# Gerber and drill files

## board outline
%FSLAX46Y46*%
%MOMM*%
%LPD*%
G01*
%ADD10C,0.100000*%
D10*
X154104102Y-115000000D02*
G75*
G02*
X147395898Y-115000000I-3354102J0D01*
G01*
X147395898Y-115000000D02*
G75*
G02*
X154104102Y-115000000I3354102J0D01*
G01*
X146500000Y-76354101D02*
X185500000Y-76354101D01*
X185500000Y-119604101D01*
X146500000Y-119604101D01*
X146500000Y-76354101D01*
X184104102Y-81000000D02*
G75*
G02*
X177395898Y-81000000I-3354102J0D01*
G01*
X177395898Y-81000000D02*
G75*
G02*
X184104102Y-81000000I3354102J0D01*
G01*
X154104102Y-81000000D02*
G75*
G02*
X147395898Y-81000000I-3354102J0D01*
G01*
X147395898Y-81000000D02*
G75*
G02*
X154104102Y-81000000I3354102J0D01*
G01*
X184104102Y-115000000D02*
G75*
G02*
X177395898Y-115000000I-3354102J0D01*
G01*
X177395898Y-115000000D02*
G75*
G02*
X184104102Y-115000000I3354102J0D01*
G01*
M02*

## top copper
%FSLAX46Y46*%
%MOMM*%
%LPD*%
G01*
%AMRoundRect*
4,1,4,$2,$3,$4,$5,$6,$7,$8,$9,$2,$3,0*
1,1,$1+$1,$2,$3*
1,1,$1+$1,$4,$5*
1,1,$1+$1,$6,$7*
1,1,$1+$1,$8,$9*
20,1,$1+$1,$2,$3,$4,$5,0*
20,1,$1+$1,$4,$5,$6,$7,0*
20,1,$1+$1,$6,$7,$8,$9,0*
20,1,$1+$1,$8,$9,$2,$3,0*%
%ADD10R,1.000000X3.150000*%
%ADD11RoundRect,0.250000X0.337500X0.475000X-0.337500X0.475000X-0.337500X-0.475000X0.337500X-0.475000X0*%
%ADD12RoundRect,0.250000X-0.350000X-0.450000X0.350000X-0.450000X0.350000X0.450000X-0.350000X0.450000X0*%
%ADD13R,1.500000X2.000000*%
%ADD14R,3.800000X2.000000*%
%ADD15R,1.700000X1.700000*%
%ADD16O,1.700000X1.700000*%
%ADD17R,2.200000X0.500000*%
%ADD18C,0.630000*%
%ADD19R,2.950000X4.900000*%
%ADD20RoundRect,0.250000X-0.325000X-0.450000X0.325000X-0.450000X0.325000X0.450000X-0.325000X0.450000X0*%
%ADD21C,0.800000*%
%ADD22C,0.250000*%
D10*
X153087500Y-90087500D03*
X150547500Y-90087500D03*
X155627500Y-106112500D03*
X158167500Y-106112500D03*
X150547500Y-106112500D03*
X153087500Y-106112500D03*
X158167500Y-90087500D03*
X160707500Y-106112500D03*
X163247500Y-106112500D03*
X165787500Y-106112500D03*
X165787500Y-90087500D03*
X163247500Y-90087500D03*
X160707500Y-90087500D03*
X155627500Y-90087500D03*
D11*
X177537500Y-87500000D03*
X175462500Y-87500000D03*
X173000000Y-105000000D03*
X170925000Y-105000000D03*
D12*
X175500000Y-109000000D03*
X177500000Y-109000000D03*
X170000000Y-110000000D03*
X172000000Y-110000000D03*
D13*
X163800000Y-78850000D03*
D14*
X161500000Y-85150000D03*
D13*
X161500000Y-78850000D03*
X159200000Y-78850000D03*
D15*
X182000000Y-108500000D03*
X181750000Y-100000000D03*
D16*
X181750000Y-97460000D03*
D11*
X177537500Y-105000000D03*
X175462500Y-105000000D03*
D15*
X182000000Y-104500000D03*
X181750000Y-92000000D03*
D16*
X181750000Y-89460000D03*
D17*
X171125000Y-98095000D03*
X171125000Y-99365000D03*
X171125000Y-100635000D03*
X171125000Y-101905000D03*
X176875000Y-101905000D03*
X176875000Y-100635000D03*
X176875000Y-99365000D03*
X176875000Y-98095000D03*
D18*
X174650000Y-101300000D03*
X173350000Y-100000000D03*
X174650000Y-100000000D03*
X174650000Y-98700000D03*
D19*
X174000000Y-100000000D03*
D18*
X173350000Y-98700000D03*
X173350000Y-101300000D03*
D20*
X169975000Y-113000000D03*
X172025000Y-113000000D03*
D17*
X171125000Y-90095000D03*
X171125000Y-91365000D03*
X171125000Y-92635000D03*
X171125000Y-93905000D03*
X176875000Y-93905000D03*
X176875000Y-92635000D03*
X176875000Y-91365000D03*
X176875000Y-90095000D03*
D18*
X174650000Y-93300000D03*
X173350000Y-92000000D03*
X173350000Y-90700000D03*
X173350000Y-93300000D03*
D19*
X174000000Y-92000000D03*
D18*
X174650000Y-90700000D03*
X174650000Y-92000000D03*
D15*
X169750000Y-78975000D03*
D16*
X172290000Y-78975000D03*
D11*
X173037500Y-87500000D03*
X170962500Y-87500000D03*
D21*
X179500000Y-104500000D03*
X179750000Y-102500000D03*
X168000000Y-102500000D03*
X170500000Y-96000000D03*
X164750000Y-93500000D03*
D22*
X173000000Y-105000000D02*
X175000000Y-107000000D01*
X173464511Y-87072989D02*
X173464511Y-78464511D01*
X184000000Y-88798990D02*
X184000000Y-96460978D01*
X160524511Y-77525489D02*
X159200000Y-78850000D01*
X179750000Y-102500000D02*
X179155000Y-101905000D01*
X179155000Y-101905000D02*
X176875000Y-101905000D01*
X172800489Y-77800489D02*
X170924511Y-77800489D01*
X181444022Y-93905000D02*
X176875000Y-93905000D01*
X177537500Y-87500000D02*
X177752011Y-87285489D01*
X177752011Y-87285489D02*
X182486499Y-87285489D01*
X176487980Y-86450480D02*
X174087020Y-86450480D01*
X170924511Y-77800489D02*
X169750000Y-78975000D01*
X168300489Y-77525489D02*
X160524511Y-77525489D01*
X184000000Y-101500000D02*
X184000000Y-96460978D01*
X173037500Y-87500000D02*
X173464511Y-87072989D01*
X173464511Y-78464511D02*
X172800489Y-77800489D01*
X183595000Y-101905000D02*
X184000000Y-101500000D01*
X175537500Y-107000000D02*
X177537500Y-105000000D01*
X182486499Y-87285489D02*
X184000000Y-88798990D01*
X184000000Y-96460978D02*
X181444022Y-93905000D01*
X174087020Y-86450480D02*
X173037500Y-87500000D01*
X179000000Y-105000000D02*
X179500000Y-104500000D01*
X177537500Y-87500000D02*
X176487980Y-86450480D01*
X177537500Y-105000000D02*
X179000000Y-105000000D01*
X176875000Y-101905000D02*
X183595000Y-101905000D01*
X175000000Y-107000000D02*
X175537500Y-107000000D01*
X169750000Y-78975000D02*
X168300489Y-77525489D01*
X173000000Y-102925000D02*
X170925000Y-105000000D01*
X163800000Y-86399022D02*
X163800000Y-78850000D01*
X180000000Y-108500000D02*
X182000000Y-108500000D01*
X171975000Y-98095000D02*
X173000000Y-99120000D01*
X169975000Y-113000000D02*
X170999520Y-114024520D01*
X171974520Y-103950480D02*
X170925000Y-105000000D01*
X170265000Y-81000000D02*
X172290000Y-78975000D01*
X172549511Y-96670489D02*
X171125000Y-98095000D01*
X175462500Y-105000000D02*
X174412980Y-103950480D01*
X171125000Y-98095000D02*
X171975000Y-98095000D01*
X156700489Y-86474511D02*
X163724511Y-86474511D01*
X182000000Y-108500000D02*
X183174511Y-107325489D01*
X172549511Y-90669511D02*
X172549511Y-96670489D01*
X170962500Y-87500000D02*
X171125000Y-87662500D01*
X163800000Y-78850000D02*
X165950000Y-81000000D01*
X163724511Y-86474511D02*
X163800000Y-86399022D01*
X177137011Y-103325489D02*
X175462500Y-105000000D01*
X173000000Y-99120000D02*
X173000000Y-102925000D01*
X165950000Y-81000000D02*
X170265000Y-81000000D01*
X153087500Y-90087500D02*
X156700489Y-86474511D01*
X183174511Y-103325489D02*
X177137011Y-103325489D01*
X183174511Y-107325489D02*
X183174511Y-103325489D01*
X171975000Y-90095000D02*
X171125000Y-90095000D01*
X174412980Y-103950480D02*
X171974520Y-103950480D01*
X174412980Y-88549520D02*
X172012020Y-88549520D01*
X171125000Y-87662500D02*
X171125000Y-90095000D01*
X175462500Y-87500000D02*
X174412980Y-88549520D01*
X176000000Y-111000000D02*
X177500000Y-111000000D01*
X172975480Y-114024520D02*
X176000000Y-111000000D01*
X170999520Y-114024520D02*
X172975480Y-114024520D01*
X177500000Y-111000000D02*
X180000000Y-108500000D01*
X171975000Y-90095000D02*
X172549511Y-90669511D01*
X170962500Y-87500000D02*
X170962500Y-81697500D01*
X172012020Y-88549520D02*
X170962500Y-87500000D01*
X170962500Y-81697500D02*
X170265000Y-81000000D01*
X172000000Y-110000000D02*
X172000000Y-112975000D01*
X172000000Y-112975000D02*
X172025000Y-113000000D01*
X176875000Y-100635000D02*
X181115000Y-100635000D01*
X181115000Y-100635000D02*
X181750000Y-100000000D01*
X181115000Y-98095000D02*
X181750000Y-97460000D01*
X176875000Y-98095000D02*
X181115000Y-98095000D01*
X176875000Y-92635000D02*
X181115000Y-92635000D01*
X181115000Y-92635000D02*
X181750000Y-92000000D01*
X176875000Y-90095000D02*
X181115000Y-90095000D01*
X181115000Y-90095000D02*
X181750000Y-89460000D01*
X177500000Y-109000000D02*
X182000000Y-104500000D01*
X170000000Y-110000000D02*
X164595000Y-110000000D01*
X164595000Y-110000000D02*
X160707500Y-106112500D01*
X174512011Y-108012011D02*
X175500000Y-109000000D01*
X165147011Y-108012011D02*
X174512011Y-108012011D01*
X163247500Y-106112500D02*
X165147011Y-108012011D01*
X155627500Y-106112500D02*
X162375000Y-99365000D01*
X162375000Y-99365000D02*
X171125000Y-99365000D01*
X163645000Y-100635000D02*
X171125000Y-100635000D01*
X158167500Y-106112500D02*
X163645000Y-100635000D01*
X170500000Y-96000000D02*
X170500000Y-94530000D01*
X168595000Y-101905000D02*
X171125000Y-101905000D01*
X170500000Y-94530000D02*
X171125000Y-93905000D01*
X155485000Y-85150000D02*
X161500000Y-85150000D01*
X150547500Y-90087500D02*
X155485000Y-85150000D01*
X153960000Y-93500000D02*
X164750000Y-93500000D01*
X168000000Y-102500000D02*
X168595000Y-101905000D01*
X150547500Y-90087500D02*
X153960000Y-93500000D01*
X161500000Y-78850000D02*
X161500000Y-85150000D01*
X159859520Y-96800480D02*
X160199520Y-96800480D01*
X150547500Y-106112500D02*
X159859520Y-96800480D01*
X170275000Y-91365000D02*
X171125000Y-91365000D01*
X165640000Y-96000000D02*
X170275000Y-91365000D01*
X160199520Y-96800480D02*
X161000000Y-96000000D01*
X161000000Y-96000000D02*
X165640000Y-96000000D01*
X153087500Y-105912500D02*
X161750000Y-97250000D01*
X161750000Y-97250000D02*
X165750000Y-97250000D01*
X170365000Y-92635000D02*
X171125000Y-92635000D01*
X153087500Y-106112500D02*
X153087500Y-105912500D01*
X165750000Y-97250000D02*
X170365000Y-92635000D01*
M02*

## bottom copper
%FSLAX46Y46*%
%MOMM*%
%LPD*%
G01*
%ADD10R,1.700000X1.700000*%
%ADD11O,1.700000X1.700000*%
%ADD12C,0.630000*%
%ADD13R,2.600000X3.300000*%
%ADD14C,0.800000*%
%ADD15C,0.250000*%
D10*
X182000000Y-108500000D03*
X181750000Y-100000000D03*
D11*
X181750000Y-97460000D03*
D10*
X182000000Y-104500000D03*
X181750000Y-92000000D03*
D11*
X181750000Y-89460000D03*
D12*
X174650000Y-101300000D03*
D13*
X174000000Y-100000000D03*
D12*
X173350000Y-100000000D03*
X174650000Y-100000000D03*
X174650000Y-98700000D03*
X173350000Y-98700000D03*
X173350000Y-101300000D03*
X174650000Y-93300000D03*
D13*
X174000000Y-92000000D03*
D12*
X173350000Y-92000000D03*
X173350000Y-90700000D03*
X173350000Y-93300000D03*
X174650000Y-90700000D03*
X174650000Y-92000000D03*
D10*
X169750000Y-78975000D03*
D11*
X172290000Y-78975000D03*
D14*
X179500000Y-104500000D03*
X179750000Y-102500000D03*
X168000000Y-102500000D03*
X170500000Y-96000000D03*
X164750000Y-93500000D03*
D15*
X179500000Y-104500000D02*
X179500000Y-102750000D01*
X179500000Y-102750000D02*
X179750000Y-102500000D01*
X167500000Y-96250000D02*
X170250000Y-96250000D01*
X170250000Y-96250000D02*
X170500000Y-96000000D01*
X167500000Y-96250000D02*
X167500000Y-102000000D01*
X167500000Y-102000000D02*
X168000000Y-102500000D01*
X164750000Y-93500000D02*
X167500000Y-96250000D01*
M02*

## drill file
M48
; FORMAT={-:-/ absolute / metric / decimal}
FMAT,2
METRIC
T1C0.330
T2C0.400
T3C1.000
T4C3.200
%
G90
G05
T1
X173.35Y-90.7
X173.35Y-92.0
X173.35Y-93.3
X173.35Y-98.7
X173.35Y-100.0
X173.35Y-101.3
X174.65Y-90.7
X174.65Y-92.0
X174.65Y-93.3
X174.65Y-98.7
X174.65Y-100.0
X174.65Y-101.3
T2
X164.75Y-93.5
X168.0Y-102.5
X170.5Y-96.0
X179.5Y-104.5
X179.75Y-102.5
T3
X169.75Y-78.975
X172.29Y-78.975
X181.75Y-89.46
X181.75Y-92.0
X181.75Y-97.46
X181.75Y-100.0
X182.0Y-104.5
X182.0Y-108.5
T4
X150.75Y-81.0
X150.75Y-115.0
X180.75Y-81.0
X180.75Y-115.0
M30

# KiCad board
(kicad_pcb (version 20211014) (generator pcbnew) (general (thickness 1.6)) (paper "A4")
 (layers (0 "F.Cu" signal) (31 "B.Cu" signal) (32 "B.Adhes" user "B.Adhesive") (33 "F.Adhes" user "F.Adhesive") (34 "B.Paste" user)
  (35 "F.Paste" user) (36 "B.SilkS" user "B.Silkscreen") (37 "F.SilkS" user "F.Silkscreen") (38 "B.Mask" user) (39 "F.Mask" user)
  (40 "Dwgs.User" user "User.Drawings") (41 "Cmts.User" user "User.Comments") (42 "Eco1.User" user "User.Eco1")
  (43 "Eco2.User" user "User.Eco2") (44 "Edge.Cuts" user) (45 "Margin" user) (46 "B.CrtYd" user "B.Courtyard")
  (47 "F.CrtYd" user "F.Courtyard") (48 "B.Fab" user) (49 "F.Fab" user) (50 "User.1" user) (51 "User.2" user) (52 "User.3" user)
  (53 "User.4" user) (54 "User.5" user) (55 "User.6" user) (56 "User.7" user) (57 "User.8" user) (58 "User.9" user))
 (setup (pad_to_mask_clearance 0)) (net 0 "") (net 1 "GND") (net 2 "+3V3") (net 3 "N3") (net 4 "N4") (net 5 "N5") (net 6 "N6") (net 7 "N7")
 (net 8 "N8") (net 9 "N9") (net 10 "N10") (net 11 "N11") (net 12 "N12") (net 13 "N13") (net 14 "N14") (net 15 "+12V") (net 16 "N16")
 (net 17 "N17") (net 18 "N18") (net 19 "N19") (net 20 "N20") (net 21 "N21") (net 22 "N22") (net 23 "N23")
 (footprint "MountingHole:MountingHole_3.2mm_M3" (layer "F.Cu") (at 180.75 115)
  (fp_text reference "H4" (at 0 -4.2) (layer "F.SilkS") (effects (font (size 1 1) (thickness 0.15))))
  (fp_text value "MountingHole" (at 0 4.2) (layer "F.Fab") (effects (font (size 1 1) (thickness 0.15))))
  (pad "" np_thru_hole circle (at 0 0) (size 3.2 3.2) (drill 3.2) (layers *.Cu *.Mask)))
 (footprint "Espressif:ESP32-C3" (layer "F.Cu") (at 159.9675 97.5125 90)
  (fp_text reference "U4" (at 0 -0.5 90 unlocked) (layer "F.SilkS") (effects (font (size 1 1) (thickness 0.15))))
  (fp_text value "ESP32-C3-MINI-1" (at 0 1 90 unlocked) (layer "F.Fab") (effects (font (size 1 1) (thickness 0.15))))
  (pad "1" smd rect (at 7.425 -6.88 90) (size 3.15 1) (layers "F.Cu" "F.Paste" "F.Mask") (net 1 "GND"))
  (pad "3" smd rect (at 7.425 -9.42 90) (size 3.15 1) (layers "F.Cu" "F.Paste" "F.Mask") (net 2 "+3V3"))
  (pad "5" smd rect (at -8.6 -4.34 90) (size 3.15 1) (layers "F.Cu" "F.Paste" "F.Mask") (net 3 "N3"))
  (pad "6" smd rect (at -8.6 -1.8 90) (size 3.15 1) (layers "F.Cu" "F.Paste" "F.Mask") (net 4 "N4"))
  (pad "12" smd rect (at -8.6 -9.42 90) (size 3.15 1) (layers "F.Cu" "F.Paste" "F.Mask") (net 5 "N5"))
  (pad "13" smd rect (at -8.6 -6.88 90) (size 3.15 1) (layers "F.Cu" "F.Paste" "F.Mask") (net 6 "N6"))
  (pad "16" smd rect (at 7.425 -1.8 90) (size 3.15 1) (layers "F.Cu" "F.Paste" "F.Mask") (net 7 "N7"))
  (pad "18" smd rect (at -8.6 0.74 90) (size 3.15 1) (layers "F.Cu" "F.Paste" "F.Mask") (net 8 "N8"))
  (pad "19" smd rect (at -8.6 3.28 90) (size 3.15 1) (layers "F.Cu" "F.Paste" "F.Mask") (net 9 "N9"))
  (pad "20" smd rect (at -8.6 5.82 90) (size 3.15 1) (layers "F.Cu" "F.Paste" "F.Mask") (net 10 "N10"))
  (pad "21" smd rect (at 7.425 5.82 90) (size 3.15 1) (layers "F.Cu" "F.Paste" "F.Mask") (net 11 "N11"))
  (pad "22" smd rect (at 7.425 3.28 90) (size 3.15 1) (layers "F.Cu" "F.Paste" "F.Mask") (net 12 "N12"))
  (pad "23" smd rect (at 7.425 0.74 90) (size 3.15 1) (layers "F.Cu" "F.Paste" "F.Mask") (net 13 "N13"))
  (pad "35" smd rect (at 7.425 -4.34 90) (size 3.15 1) (layers "F.Cu" "F.Paste" "F.Mask") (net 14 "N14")))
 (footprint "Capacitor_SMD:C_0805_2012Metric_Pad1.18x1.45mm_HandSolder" (layer "F.Cu") (at 176.5 87.5 180)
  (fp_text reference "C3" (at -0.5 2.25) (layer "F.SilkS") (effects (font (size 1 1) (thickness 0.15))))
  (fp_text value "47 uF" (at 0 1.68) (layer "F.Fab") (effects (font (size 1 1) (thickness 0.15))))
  (pad "1" smd roundrect (at -1.0375 0 180) (size 1.175 1.45) (layers "F.Cu" "F.Paste" "F.Mask") (roundrect_rratio 0.2127659574)
   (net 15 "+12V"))
  (pad "2" smd roundrect (at 1.0375 0 180) (size 1.175 1.45) (layers "F.Cu" "F.Paste" "F.Mask") (roundrect_rratio 0.2127659574)
   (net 1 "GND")))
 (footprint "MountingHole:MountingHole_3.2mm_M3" (layer "F.Cu") (at 180.75 81)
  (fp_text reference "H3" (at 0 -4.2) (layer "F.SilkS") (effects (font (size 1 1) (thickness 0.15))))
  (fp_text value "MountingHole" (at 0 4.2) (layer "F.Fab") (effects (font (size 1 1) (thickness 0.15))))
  (pad "" np_thru_hole circle (at 0 0) (size 3.2 3.2) (drill 3.2) (layers *.Cu *.Mask)))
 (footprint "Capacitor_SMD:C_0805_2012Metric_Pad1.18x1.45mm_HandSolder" (layer "F.Cu") (at 171.9625 105 180)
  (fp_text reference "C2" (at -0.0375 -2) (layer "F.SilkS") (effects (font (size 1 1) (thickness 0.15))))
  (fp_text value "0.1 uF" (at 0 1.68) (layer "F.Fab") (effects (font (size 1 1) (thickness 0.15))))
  (pad "1" smd roundrect (at -1.0375 0 180) (size 1.175 1.45) (layers "F.Cu" "F.Paste" "F.Mask") (roundrect_rratio 0.2127659574)
   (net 15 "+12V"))
  (pad "2" smd roundrect (at 1.0375 0 180) (size 1.175 1.45) (layers "F.Cu" "F.Paste" "F.Mask") (roundrect_rratio 0.2127659574)
   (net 1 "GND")))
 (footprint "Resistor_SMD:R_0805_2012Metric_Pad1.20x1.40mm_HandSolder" (layer "F.Cu") (at 176.5 109)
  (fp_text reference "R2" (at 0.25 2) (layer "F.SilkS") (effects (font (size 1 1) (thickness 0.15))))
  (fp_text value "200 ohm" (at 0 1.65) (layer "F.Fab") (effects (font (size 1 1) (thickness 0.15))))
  (pad "1" smd roundrect (at -1 0) (size 1.2 1.4) (layers "F.Cu" "F.Paste" "F.Mask") (roundrect_rratio 0.2083333333) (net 9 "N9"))
  (pad "2" smd roundrect (at 1 0) (size 1.2 1.4) (layers "F.Cu" "F.Paste" "F.Mask") (roundrect_rratio 0.2083333333) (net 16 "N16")))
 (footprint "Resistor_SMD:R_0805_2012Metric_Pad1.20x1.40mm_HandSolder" (layer "F.Cu") (at 171 110)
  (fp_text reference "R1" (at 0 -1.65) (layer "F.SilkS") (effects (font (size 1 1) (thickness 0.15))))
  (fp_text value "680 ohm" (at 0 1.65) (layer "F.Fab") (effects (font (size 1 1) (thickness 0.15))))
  (pad "1" smd roundrect (at -1 0) (size 1.2 1.4) (layers "F.Cu" "F.Paste" "F.Mask") (roundrect_rratio 0.2083333333) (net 8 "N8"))
  (pad "2" smd roundrect (at 1 0) (size 1.2 1.4) (layers "F.Cu" "F.Paste" "F.Mask") (roundrect_rratio 0.2083333333) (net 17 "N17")))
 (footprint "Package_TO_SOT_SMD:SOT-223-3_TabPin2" (layer "F.Cu") (at 161.5 82 -90)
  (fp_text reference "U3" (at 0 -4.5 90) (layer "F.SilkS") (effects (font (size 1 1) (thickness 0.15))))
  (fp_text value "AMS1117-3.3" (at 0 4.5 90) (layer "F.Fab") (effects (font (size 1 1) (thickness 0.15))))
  (pad "1" smd rect (at -3.15 -2.3 270) (size 2 1.5) (layers "F.Cu" "F.Paste" "F.Mask") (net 1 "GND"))
  (pad "2" smd rect (at 3.15 0 270) (size 2 3.8) (layers "F.Cu" "F.Paste" "F.Mask") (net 2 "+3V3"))
  (pad "2" smd rect (at -3.15 0 270) (size 2 1.5) (layers "F.Cu" "F.Paste" "F.Mask") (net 2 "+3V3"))
  (pad "3" smd rect (at -3.15 2.3 270) (size 2 1.5) (layers "F.Cu" "F.Paste" "F.Mask") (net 15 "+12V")))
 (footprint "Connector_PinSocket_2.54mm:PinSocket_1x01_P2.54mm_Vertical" (layer "F.Cu") (at 182 108.5 180)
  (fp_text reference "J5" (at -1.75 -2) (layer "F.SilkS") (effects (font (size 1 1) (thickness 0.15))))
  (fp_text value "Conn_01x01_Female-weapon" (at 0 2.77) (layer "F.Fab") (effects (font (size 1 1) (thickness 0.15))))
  (pad "1" thru_hole rect (at 0 0 180) (size 1.7 1.7) (drill 1) (layers *.Cu *.Mask) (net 1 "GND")))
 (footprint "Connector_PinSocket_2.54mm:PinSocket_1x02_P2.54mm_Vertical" (layer "F.Cu") (at 181.75 100 180)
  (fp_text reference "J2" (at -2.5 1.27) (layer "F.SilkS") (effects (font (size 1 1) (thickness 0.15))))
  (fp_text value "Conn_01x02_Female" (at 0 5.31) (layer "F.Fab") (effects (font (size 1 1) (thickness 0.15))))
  (pad "1" thru_hole rect (at 0 0 180) (size 1.7 1.7) (drill 1) (layers *.Cu *.Mask) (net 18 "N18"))
  (pad "2" thru_hole oval (at 0 2.54 180) (size 1.7 1.7) (drill 1) (layers *.Cu *.Mask) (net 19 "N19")))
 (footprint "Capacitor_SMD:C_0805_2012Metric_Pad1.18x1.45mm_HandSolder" (layer "F.Cu") (at 176.5 105 180)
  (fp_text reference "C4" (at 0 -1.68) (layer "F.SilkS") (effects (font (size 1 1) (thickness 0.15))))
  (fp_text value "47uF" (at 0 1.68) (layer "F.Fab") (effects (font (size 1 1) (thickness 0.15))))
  (pad "1" smd roundrect (at -1.0375 0 180) (size 1.175 1.45) (layers "F.Cu" "F.Paste" "F.Mask") (roundrect_rratio 0.2127659574)
   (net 15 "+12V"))
  (pad "2" smd roundrect (at 1.0375 0 180) (size 1.175 1.45) (layers "F.Cu" "F.Paste" "F.Mask") (roundrect_rratio 0.2127659574)
   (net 1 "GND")))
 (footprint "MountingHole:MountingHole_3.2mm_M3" (layer "F.Cu") (at 150.75 115)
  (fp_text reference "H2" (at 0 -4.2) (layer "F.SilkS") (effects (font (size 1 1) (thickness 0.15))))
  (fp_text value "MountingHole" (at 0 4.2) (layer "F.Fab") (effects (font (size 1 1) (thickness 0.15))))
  (pad "" np_thru_hole circle (at 0 0) (size 3.2 3.2) (drill 3.2) (layers *.Cu *.Mask)))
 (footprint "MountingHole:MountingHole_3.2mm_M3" (layer "F.Cu") (at 150.75 81)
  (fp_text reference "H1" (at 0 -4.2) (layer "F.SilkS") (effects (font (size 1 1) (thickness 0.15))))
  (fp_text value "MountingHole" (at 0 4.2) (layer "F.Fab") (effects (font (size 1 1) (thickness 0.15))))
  (pad "" np_thru_hole circle (at 0 0) (size 3.2 3.2) (drill 3.2) (layers *.Cu *.Mask)))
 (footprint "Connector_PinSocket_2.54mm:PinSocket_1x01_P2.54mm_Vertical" (layer "F.Cu") (at 182 104.5)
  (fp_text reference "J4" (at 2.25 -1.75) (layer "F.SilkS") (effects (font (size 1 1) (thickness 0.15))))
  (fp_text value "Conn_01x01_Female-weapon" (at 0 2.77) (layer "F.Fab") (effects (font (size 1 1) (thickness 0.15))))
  (pad "1" thru_hole rect (at 0 0) (size 1.7 1.7) (drill 1) (layers *.Cu *.Mask) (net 16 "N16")))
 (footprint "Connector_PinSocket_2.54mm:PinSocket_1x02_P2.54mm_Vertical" (layer "F.Cu") (at 181.75 92 180)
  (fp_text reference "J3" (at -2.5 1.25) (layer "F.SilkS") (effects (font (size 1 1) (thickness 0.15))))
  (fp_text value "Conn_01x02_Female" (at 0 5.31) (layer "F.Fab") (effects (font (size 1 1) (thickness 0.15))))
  (pad "1" thru_hole rect (at 0 0 180) (size 1.7 1.7) (drill 1) (layers *.Cu *.Mask) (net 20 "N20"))
  (pad "2" thru_hole oval (at 0 2.54 180) (size 1.7 1.7) (drill 1) (layers *.Cu *.Mask) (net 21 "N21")))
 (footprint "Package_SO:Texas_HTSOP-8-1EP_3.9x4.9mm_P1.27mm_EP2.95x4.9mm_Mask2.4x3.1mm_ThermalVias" (layer "F.Cu") (at 174 100)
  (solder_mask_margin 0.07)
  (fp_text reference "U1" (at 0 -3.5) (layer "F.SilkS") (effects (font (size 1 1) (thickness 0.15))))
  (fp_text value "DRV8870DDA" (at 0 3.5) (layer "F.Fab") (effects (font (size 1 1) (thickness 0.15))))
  (pad "" smd rect (at 0 0) (size 2.4 3.1) (layers "F.Paste")) (pad "" smd rect (at 0 0) (size 2.4 3.1) (layers "F.Mask"))
  (pad "1" smd rect (at -2.875 -1.905) (size 2.2 0.5) (layers "F.Cu" "F.Paste" "F.Mask") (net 1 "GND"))
  (pad "2" smd rect (at -2.875 -0.635) (size 2.2 0.5) (layers "F.Cu" "F.Paste" "F.Mask") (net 3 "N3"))
  (pad "3" smd rect (at -2.875 0.635) (size 2.2 0.5) (layers "F.Cu" "F.Paste" "F.Mask") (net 4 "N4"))
  (pad "4" smd rect (at -2.875 1.905) (size 2.2 0.5) (layers "F.Cu" "F.Paste" "F.Mask") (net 2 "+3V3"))
  (pad "5" smd rect (at 2.875 1.905) (size 2.2 0.5) (layers "F.Cu" "F.Paste" "F.Mask") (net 15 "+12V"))
  (pad "6" smd rect (at 2.875 0.635) (size 2.2 0.5) (layers "F.Cu" "F.Paste" "F.Mask") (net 18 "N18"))
  (pad "7" smd rect (at 2.875 -0.635) (size 2.2 0.5) (layers "F.Cu" "F.Paste" "F.Mask") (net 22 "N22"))
  (pad "8" smd rect (at 2.875 -1.905) (size 2.2 0.5) (layers "F.Cu" "F.Paste" "F.Mask") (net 19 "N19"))
  (pad "9" thru_hole circle (at 0.65 1.3) (size 0.63 0.63) (drill 0.33) (layers *.Cu *.Mask) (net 1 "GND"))
  (pad "9" smd rect (at 0 0) (size 2.6 3.3) (layers "B.Cu") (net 1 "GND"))
  (pad "9" thru_hole circle (at -0.65 0) (size 0.63 0.63) (drill 0.33) (layers *.Cu *.Mask) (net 1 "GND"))
  (pad "9" thru_hole circle (at 0.65 0) (size 0.63 0.63) (drill 0.33) (layers *.Cu *.Mask) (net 1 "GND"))
  (pad "9" thru_hole circle (at 0.65 -1.3) (size 0.63 0.63) (drill 0.33) (layers *.Cu *.Mask) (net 1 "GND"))
  (pad "9" smd rect (at 0 0) (size 2.95 4.9) (layers "F.Cu") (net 1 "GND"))
  (pad "9" thru_hole circle (at -0.65 -1.3) (size 0.63 0.63) (drill 0.33) (layers *.Cu *.Mask) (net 1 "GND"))
  (pad "9" thru_hole circle (at -0.65 1.3) (size 0.63 0.63) (drill 0.33) (layers *.Cu *.Mask) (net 1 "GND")))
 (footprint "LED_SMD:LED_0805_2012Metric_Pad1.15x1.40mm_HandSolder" (layer "F.Cu") (at 171 113)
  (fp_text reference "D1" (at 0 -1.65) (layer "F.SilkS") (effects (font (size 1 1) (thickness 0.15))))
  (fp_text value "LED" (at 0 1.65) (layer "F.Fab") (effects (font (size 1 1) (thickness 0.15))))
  (pad "1" smd roundrect (at -1.025 0) (size 1.15 1.4) (layers "F.Cu" "F.Paste" "F.Mask") (roundrect_rratio 0.2173913043) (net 1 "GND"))
  (pad "2" smd roundrect (at 1.025 0) (size 1.15 1.4) (layers "F.Cu" "F.Paste" "F.Mask") (roundrect_rratio 0.2173913043) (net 17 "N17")))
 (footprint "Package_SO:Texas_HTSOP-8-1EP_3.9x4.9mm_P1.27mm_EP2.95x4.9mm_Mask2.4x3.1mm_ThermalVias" (layer "F.Cu") (at 174 92)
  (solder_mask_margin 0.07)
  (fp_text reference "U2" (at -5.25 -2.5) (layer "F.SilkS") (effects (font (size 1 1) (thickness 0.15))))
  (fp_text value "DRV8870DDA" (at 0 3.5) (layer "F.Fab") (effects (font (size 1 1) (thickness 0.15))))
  (pad "" smd rect (at 0 0) (size 2.4 3.1) (layers "F.Mask")) (pad "" smd rect (at 0 0) (size 2.4 3.1) (layers "F.Paste"))
  (pad "1" smd rect (at -2.875 -1.905) (size 2.2 0.5) (layers "F.Cu" "F.Paste" "F.Mask") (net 1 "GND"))
  (pad "2" smd rect (at -2.875 -0.635) (size 2.2 0.5) (layers "F.Cu" "F.Paste" "F.Mask") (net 5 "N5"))
  (pad "3" smd rect (at -2.875 0.635) (size 2.2 0.5) (layers "F.Cu" "F.Paste" "F.Mask") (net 6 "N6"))
  (pad "4" smd rect (at -2.875 1.905) (size 2.2 0.5) (layers "F.Cu" "F.Paste" "F.Mask") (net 2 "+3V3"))
  (pad "5" smd rect (at 2.875 1.905) (size 2.2 0.5) (layers "F.Cu" "F.Paste" "F.Mask") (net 15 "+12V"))
  (pad "6" smd rect (at 2.875 0.635) (size 2.2 0.5) (layers "F.Cu" "F.Paste" "F.Mask") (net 20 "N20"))
  (pad "7" smd rect (at 2.875 -0.635) (size 2.2 0.5) (layers "F.Cu" "F.Paste" "F.Mask") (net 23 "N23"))
  (pad "8" smd rect (at 2.875 -1.905) (size 2.2 0.5) (layers "F.Cu" "F.Paste" "F.Mask") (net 21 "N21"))
  (pad "9" thru_hole circle (at 0.65 1.3) (size 0.63 0.63) (drill 0.33) (layers *.Cu *.Mask) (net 1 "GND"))
  (pad "9" smd rect (at 0 0) (size 2.6 3.3) (layers "B.Cu") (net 1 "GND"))
  (pad "9" thru_hole circle (at -0.65 0) (size 0.63 0.63) (drill 0.33) (layers *.Cu *.Mask) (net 1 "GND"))
  (pad "9" thru_hole circle (at -0.65 -1.3) (size 0.63 0.63) (drill 0.33) (layers *.Cu *.Mask) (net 1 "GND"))
  (pad "9" thru_hole circle (at -0.65 1.3) (size 0.63 0.63) (drill 0.33) (layers *.Cu *.Mask) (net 1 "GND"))
  (pad "9" smd rect (at 0 0) (size 2.95 4.9) (layers "F.Cu") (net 1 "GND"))
  (pad "9" thru_hole circle (at 0.65 -1.3) (size 0.63 0.63) (drill 0.33) (layers *.Cu *.Mask) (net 1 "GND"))
  (pad "9" thru_hole circle (at 0.65 0) (size 0.63 0.63) (drill 0.33) (layers *.Cu *.Mask) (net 1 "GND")))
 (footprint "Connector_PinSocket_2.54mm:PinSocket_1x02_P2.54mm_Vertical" (layer "F.Cu") (at 169.75 78.975 90)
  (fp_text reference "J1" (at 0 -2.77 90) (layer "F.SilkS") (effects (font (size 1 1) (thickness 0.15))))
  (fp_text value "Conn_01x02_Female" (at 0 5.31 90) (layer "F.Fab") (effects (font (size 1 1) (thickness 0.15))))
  (pad "1" thru_hole rect (at 0 0 90) (size 1.7 1.7) (drill 1) (layers *.Cu *.Mask) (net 15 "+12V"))
  (pad "2" thru_hole oval (at 0 2.54 90) (size 1.7 1.7) (drill 1) (layers *.Cu *.Mask) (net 1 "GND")))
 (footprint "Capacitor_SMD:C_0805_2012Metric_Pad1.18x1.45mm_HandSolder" (layer "F.Cu") (at 172 87.5 180)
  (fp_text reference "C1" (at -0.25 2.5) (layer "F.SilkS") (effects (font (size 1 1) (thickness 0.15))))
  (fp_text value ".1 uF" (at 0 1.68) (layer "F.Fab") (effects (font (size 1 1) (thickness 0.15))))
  (pad "1" smd roundrect (at -1.0375 0 180) (size 1.175 1.45) (layers "F.Cu" "F.Paste" "F.Mask") (roundrect_rratio 0.2127659574)
   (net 15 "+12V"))
  (pad "2" smd roundrect (at 1.0375 0 180) (size 1.175 1.45) (layers "F.Cu" "F.Paste" "F.Mask") (roundrect_rratio 0.2127659574)
   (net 1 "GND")))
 (gr_circle (center 150.75 115) (end 153.75 116.5) (layer "Edge.Cuts") (width 0.1) (fill none))
 (gr_rect (start 146.5 76.354101) (end 185.5 119.604101) (layer "Edge.Cuts") (width 0.1) (fill none))
 (gr_circle (center 180.75 81) (end 183.75 82.5) (layer "Edge.Cuts") (width 0.1) (fill none))
 (gr_circle (center 150.75 81) (end 153.75 82.5) (layer "Edge.Cuts") (width 0.1) (fill none))
 (gr_circle (center 180.75 115) (end 183.75 116.5) (layer "Edge.Cuts") (width 0.1) (fill none))
 (segment (start 173 105) (end 175 107) (width 0.25) (layer "F.Cu") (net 15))
 (segment (start 173.464511 87.072989) (end 173.464511 78.464511) (width 0.25) (layer "F.Cu") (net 15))
 (segment (start 184 88.79899) (end 184 96.460978) (width 0.25) (layer "F.Cu") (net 15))
 (segment (start 160.524511 77.525489) (end 159.2 78.85) (width 0.25) (layer "F.Cu") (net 15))
 (segment (start 179.75 102.5) (end 179.155 101.905) (width 0.25) (layer "F.Cu") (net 15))
 (segment (start 179.155 101.905) (end 176.875 101.905) (width 0.25) (layer "F.Cu") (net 15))
 (segment (start 172.800489 77.800489) (end 170.924511 77.800489) (width 0.25) (layer "F.Cu") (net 15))
 (segment (start 181.444022 93.905) (end 176.875 93.905) (width 0.25) (layer "F.Cu") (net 15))
 (segment (start 177.5375 87.5) (end 177.752011 87.285489) (width 0.25) (layer "F.Cu") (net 15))
 (segment (start 177.752011 87.285489) (end 182.486499 87.285489) (width 0.25) (layer "F.Cu") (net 15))
 (segment (start 176.48798 86.45048) (end 174.08702 86.45048) (width 0.25) (layer "F.Cu") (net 15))
 (segment (start 170.924511 77.800489) (end 169.75 78.975) (width 0.25) (layer "F.Cu") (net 15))
 (segment (start 168.300489 77.525489) (end 160.524511 77.525489) (width 0.25) (layer "F.Cu") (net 15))
 (segment (start 184 101.5) (end 184 96.460978) (width 0.25) (layer "F.Cu") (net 15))
 (segment (start 173.0375 87.5) (end 173.464511 87.072989) (width 0.25) (layer "F.Cu") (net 15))
 (segment (start 173.464511 78.464511) (end 172.800489 77.800489) (width 0.25) (layer "F.Cu") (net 15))
 (segment (start 183.595 101.905) (end 184 101.5) (width 0.25) (layer "F.Cu") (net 15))
 (segment (start 175.5375 107) (end 177.5375 105) (width 0.25) (layer "F.Cu") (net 15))
 (segment (start 182.486499 87.285489) (end 184 88.79899) (width 0.25) (layer "F.Cu") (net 15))
 (segment (start 184 96.460978) (end 181.444022 93.905) (width 0.25) (layer "F.Cu") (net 15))
 (segment (start 174.08702 86.45048) (end 173.0375 87.5) (width 0.25) (layer "F.Cu") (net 15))
 (segment (start 179 105) (end 179.5 104.5) (width 0.25) (layer "F.Cu") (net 15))
 (segment (start 177.5375 87.5) (end 176.48798 86.45048) (width 0.25) (layer "F.Cu") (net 15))
 (segment (start 177.5375 105) (end 179 105) (width 0.25) (layer "F.Cu") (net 15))
 (segment (start 176.875 101.905) (end 183.595 101.905) (width 0.25) (layer "F.Cu") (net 15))
 (segment (start 175 107) (end 175.5375 107) (width 0.25) (layer "F.Cu") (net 15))
 (segment (start 169.75 78.975) (end 168.300489 77.525489) (width 0.25) (layer "F.Cu") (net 15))
 (via (at 179.5 104.5) (size 0.8) (drill 0.4) (layers "F.Cu" "B.Cu") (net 15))
 (via (at 179.75 102.5) (size 0.8) (drill 0.4) (layers "F.Cu" "B.Cu") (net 15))
 (segment (start 179.5 104.5) (end 179.5 102.75) (width 0.25) (layer "B.Cu") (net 15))
 (segment (start 179.5 102.75) (end 179.75 102.5) (width 0.25) (layer "B.Cu") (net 15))
 (segment (start 173 102.925) (end 170.925 105) (width 0.25) (layer "F.Cu") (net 1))
 (segment (start 163.8 86.399022) (end 163.8 78.85) (width 0.25) (layer "F.Cu") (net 1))
 (segment (start 180 108.5) (end 182 108.5) (width 0.25) (layer "F.Cu") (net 1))
 (segment (start 171.975 98.095) (end 173 99.12) (width 0.25) (layer "F.Cu") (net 1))
 (segment (start 169.975 113) (end 170.99952 114.02452) (width 0.25) (layer "F.Cu") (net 1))
 (segment (start 171.97452 103.95048) (end 170.925 105) (width 0.25) (layer "F.Cu") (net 1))
 (segment (start 170.265 81) (end 172.29 78.975) (width 0.25) (layer "F.Cu") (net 1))
 (segment (start 172.549511 96.670489) (end 171.125 98.095) (width 0.25) (layer "F.Cu") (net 1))
 (segment (start 175.4625 105) (end 174.41298 103.95048) (width 0.25) (layer "F.Cu") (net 1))
 (segment (start 171.125 98.095) (end 171.975 98.095) (width 0.25) (layer "F.Cu") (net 1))
 (segment (start 156.700489 86.474511) (end 163.724511 86.474511) (width 0.25) (layer "F.Cu") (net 1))
 (segment (start 182 108.5) (end 183.174511 107.325489) (width 0.25) (layer "F.Cu") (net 1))
 (segment (start 172.549511 90.669511) (end 172.549511 96.670489) (width 0.25) (layer "F.Cu") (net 1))
 (segment (start 170.9625 87.5) (end 171.125 87.6625) (width 0.25) (layer "F.Cu") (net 1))
 (segment (start 163.8 78.85) (end 165.95 81) (width 0.25) (layer "F.Cu") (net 1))
 (segment (start 163.724511 86.474511) (end 163.8 86.399022) (width 0.25) (layer "F.Cu") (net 1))
 (segment (start 177.137011 103.325489) (end 175.4625 105) (width 0.25) (layer "F.Cu") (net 1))
 (segment (start 173 99.12) (end 173 102.925) (width 0.25) (layer "F.Cu") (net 1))
 (segment (start 165.95 81) (end 170.265 81) (width 0.25) (layer "F.Cu") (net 1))
 (segment (start 153.0875 90.0875) (end 156.700489 86.474511) (width 0.25) (layer "F.Cu") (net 1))
 (segment (start 183.174511 103.325489) (end 177.137011 103.325489) (width 0.25) (layer "F.Cu") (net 1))
 (segment (start 183.174511 107.325489) (end 183.174511 103.325489) (width 0.25) (layer "F.Cu") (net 1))
 (segment (start 171.975 90.095) (end 171.125 90.095) (width 0.25) (layer "F.Cu") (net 1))
 (segment (start 174.41298 103.95048) (end 171.97452 103.95048) (width 0.25) (layer "F.Cu") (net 1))
 (segment (start 174.41298 88.54952) (end 172.01202 88.54952) (width 0.25) (layer "F.Cu") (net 1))
 (segment (start 171.125 87.6625) (end 171.125 90.095) (width 0.25) (layer "F.Cu") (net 1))
 (segment (start 175.4625 87.5) (end 174.41298 88.54952) (width 0.25) (layer "F.Cu") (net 1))
 (segment (start 176 111) (end 177.5 111) (width 0.25) (layer "F.Cu") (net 1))
 (segment (start 172.97548 114.02452) (end 176 111) (width 0.25) (layer "F.Cu") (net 1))
 (segment (start 170.99952 114.02452) (end 172.97548 114.02452) (width 0.25) (layer "F.Cu") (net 1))
 (segment (start 177.5 111) (end 180 108.5) (width 0.25) (layer "F.Cu") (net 1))
 (segment (start 171.975 90.095) (end 172.549511 90.669511) (width 0.25) (layer "F.Cu") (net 1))
 (segment (start 170.9625 87.5) (end 170.9625 81.6975) (width 0.25) (layer "F.Cu") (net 1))
 (segment (start 172.01202 88.54952) (end 170.9625 87.5) (width 0.25) (layer "F.Cu") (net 1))
 (segment (start 170.9625 81.6975) (end 170.265 81) (width 0.25) (layer "F.Cu") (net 1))
 (segment (start 172 110) (end 172 112.975) (width 0.25) (layer "F.Cu") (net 17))
 (segment (start 172 112.975) (end 172.025 113) (width 0.25) (layer "F.Cu") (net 17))
 (segment (start 176.875 100.635) (end 181.115 100.635) (width 0.25) (layer "F.Cu") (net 18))
 (segment (start 181.115 100.635) (end 181.75 100) (width 0.25) (layer "F.Cu") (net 18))
 (segment (start 181.115 98.095) (end 181.75 97.46) (width 0.25) (layer "F.Cu") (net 19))
 (segment (start 176.875 98.095) (end 181.115 98.095) (width 0.25) (layer "F.Cu") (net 19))
 (segment (start 176.875 92.635) (end 181.115 92.635) (width 0.25) (layer "F.Cu") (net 20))
 (segment (start 181.115 92.635) (end 181.75 92) (width 0.25) (layer "F.Cu") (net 20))
 (segment (start 176.875 90.095) (end 181.115 90.095) (width 0.25) (layer "F.Cu") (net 21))
 (segment (start 181.115 90.095) (end 181.75 89.46) (width 0.25) (layer "F.Cu") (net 21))
 (segment (start 177.5 109) (end 182 104.5) (width 0.25) (layer "F.Cu") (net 16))
 (segment (start 170 110) (end 164.595 110) (width 0.25) (layer "F.Cu") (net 8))
 (segment (start 164.595 110) (end 160.7075 106.1125) (width 0.25) (layer "F.Cu") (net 8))
 (segment (start 174.512011 108.012011) (end 175.5 109) (width 0.25) (layer "F.Cu") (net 9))
 (segment (start 165.147011 108.012011) (end 174.512011 108.012011) (width 0.25) (layer "F.Cu") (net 9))
 (segment (start 163.2475 106.1125) (end 165.147011 108.012011) (width 0.25) (layer "F.Cu") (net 9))
 (segment (start 155.6275 106.1125) (end 162.375 99.365) (width 0.25) (layer "F.Cu") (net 3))
 (segment (start 162.375 99.365) (end 171.125 99.365) (width 0.25) (layer "F.Cu") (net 3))
 (segment (start 163.645 100.635) (end 171.125 100.635) (width 0.25) (layer "F.Cu") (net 4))
 (segment (start 158.1675 106.1125) (end 163.645 100.635) (width 0.25) (layer "F.Cu") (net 4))
 (segment (start 170.5 96) (end 170.5 94.53) (width 0.25) (layer "F.Cu") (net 2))
 (segment (start 168.595 101.905) (end 171.125 101.905) (width 0.25) (layer "F.Cu") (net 2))
 (segment (start 170.5 94.53) (end 171.125 93.905) (width 0.25) (layer "F.Cu") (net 2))
 (segment (start 155.485 85.15) (end 161.5 85.15) (width 0.25) (layer "F.Cu") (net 2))
 (segment (start 150.5475 90.0875) (end 155.485 85.15) (width 0.25) (layer "F.Cu") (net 2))
 (segment (start 153.96 93.5) (end 164.75 93.5) (width 0.25) (layer "F.Cu") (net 2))
 (segment (start 168 102.5) (end 168.595 101.905) (width 0.25) (layer "F.Cu") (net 2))
 (segment (start 150.5475 90.0875) (end 153.96 93.5) (width 0.25) (layer "F.Cu") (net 2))
 (segment (start 161.5 78.85) (end 161.5 85.15) (width 0.25) (layer "F.Cu") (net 2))
 (via (at 168 102.5) (size 0.8) (drill 0.4) (layers "F.Cu" "B.Cu") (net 2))
 (via (at 170.5 96) (size 0.8) (drill 0.4) (layers "F.Cu" "B.Cu") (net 2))
 (via (at 164.75 93.5) (size 0.8) (drill 0.4) (layers "F.Cu" "B.Cu") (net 2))
 (segment (start 167.5 96.25) (end 170.25 96.25) (width 0.25) (layer "B.Cu") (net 2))
 (segment (start 170.25 96.25) (end 170.5 96) (width 0.25) (layer "B.Cu") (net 2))
 (segment (start 167.5 96.25) (end 167.5 102) (width 0.25) (layer "B.Cu") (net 2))
 (segment (start 167.5 102) (end 168 102.5) (width 0.25) (layer "B.Cu") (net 2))
 (segment (start 164.75 93.5) (end 167.5 96.25) (width 0.25) (layer "B.Cu") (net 2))
 (segment (start 159.85952 96.80048) (end 160.19952 96.80048) (width 0.25) (layer "F.Cu") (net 5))
 (segment (start 150.5475 106.1125) (end 159.85952 96.80048) (width 0.25) (layer "F.Cu") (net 5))
 (segment (start 170.275 91.365) (end 171.125 91.365) (width 0.25) (layer "F.Cu") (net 5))
 (segment (start 165.64 96) (end 170.275 91.365) (width 0.25) (layer "F.Cu") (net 5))
 (segment (start 160.19952 96.80048) (end 161 96) (width 0.25) (layer "F.Cu") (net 5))
 (segment (start 161 96) (end 165.64 96) (width 0.25) (layer "F.Cu") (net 5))
 (segment (start 153.0875 105.9125) (end 161.75 97.25) (width 0.25) (layer "F.Cu") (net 6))
 (segment (start 161.75 97.25) (end 165.75 97.25) (width 0.25) (layer "F.Cu") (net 6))
 (segment (start 170.365 92.635) (end 171.125 92.635) (width 0.25) (layer "F.Cu") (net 6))
 (segment (start 153.0875 106.1125) (end 153.0875 105.9125) (width 0.25) (layer "F.Cu") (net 6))
 (segment (start 165.75 97.25) (end 170.365 92.635) (width 0.25) (layer "F.Cu") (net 6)))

